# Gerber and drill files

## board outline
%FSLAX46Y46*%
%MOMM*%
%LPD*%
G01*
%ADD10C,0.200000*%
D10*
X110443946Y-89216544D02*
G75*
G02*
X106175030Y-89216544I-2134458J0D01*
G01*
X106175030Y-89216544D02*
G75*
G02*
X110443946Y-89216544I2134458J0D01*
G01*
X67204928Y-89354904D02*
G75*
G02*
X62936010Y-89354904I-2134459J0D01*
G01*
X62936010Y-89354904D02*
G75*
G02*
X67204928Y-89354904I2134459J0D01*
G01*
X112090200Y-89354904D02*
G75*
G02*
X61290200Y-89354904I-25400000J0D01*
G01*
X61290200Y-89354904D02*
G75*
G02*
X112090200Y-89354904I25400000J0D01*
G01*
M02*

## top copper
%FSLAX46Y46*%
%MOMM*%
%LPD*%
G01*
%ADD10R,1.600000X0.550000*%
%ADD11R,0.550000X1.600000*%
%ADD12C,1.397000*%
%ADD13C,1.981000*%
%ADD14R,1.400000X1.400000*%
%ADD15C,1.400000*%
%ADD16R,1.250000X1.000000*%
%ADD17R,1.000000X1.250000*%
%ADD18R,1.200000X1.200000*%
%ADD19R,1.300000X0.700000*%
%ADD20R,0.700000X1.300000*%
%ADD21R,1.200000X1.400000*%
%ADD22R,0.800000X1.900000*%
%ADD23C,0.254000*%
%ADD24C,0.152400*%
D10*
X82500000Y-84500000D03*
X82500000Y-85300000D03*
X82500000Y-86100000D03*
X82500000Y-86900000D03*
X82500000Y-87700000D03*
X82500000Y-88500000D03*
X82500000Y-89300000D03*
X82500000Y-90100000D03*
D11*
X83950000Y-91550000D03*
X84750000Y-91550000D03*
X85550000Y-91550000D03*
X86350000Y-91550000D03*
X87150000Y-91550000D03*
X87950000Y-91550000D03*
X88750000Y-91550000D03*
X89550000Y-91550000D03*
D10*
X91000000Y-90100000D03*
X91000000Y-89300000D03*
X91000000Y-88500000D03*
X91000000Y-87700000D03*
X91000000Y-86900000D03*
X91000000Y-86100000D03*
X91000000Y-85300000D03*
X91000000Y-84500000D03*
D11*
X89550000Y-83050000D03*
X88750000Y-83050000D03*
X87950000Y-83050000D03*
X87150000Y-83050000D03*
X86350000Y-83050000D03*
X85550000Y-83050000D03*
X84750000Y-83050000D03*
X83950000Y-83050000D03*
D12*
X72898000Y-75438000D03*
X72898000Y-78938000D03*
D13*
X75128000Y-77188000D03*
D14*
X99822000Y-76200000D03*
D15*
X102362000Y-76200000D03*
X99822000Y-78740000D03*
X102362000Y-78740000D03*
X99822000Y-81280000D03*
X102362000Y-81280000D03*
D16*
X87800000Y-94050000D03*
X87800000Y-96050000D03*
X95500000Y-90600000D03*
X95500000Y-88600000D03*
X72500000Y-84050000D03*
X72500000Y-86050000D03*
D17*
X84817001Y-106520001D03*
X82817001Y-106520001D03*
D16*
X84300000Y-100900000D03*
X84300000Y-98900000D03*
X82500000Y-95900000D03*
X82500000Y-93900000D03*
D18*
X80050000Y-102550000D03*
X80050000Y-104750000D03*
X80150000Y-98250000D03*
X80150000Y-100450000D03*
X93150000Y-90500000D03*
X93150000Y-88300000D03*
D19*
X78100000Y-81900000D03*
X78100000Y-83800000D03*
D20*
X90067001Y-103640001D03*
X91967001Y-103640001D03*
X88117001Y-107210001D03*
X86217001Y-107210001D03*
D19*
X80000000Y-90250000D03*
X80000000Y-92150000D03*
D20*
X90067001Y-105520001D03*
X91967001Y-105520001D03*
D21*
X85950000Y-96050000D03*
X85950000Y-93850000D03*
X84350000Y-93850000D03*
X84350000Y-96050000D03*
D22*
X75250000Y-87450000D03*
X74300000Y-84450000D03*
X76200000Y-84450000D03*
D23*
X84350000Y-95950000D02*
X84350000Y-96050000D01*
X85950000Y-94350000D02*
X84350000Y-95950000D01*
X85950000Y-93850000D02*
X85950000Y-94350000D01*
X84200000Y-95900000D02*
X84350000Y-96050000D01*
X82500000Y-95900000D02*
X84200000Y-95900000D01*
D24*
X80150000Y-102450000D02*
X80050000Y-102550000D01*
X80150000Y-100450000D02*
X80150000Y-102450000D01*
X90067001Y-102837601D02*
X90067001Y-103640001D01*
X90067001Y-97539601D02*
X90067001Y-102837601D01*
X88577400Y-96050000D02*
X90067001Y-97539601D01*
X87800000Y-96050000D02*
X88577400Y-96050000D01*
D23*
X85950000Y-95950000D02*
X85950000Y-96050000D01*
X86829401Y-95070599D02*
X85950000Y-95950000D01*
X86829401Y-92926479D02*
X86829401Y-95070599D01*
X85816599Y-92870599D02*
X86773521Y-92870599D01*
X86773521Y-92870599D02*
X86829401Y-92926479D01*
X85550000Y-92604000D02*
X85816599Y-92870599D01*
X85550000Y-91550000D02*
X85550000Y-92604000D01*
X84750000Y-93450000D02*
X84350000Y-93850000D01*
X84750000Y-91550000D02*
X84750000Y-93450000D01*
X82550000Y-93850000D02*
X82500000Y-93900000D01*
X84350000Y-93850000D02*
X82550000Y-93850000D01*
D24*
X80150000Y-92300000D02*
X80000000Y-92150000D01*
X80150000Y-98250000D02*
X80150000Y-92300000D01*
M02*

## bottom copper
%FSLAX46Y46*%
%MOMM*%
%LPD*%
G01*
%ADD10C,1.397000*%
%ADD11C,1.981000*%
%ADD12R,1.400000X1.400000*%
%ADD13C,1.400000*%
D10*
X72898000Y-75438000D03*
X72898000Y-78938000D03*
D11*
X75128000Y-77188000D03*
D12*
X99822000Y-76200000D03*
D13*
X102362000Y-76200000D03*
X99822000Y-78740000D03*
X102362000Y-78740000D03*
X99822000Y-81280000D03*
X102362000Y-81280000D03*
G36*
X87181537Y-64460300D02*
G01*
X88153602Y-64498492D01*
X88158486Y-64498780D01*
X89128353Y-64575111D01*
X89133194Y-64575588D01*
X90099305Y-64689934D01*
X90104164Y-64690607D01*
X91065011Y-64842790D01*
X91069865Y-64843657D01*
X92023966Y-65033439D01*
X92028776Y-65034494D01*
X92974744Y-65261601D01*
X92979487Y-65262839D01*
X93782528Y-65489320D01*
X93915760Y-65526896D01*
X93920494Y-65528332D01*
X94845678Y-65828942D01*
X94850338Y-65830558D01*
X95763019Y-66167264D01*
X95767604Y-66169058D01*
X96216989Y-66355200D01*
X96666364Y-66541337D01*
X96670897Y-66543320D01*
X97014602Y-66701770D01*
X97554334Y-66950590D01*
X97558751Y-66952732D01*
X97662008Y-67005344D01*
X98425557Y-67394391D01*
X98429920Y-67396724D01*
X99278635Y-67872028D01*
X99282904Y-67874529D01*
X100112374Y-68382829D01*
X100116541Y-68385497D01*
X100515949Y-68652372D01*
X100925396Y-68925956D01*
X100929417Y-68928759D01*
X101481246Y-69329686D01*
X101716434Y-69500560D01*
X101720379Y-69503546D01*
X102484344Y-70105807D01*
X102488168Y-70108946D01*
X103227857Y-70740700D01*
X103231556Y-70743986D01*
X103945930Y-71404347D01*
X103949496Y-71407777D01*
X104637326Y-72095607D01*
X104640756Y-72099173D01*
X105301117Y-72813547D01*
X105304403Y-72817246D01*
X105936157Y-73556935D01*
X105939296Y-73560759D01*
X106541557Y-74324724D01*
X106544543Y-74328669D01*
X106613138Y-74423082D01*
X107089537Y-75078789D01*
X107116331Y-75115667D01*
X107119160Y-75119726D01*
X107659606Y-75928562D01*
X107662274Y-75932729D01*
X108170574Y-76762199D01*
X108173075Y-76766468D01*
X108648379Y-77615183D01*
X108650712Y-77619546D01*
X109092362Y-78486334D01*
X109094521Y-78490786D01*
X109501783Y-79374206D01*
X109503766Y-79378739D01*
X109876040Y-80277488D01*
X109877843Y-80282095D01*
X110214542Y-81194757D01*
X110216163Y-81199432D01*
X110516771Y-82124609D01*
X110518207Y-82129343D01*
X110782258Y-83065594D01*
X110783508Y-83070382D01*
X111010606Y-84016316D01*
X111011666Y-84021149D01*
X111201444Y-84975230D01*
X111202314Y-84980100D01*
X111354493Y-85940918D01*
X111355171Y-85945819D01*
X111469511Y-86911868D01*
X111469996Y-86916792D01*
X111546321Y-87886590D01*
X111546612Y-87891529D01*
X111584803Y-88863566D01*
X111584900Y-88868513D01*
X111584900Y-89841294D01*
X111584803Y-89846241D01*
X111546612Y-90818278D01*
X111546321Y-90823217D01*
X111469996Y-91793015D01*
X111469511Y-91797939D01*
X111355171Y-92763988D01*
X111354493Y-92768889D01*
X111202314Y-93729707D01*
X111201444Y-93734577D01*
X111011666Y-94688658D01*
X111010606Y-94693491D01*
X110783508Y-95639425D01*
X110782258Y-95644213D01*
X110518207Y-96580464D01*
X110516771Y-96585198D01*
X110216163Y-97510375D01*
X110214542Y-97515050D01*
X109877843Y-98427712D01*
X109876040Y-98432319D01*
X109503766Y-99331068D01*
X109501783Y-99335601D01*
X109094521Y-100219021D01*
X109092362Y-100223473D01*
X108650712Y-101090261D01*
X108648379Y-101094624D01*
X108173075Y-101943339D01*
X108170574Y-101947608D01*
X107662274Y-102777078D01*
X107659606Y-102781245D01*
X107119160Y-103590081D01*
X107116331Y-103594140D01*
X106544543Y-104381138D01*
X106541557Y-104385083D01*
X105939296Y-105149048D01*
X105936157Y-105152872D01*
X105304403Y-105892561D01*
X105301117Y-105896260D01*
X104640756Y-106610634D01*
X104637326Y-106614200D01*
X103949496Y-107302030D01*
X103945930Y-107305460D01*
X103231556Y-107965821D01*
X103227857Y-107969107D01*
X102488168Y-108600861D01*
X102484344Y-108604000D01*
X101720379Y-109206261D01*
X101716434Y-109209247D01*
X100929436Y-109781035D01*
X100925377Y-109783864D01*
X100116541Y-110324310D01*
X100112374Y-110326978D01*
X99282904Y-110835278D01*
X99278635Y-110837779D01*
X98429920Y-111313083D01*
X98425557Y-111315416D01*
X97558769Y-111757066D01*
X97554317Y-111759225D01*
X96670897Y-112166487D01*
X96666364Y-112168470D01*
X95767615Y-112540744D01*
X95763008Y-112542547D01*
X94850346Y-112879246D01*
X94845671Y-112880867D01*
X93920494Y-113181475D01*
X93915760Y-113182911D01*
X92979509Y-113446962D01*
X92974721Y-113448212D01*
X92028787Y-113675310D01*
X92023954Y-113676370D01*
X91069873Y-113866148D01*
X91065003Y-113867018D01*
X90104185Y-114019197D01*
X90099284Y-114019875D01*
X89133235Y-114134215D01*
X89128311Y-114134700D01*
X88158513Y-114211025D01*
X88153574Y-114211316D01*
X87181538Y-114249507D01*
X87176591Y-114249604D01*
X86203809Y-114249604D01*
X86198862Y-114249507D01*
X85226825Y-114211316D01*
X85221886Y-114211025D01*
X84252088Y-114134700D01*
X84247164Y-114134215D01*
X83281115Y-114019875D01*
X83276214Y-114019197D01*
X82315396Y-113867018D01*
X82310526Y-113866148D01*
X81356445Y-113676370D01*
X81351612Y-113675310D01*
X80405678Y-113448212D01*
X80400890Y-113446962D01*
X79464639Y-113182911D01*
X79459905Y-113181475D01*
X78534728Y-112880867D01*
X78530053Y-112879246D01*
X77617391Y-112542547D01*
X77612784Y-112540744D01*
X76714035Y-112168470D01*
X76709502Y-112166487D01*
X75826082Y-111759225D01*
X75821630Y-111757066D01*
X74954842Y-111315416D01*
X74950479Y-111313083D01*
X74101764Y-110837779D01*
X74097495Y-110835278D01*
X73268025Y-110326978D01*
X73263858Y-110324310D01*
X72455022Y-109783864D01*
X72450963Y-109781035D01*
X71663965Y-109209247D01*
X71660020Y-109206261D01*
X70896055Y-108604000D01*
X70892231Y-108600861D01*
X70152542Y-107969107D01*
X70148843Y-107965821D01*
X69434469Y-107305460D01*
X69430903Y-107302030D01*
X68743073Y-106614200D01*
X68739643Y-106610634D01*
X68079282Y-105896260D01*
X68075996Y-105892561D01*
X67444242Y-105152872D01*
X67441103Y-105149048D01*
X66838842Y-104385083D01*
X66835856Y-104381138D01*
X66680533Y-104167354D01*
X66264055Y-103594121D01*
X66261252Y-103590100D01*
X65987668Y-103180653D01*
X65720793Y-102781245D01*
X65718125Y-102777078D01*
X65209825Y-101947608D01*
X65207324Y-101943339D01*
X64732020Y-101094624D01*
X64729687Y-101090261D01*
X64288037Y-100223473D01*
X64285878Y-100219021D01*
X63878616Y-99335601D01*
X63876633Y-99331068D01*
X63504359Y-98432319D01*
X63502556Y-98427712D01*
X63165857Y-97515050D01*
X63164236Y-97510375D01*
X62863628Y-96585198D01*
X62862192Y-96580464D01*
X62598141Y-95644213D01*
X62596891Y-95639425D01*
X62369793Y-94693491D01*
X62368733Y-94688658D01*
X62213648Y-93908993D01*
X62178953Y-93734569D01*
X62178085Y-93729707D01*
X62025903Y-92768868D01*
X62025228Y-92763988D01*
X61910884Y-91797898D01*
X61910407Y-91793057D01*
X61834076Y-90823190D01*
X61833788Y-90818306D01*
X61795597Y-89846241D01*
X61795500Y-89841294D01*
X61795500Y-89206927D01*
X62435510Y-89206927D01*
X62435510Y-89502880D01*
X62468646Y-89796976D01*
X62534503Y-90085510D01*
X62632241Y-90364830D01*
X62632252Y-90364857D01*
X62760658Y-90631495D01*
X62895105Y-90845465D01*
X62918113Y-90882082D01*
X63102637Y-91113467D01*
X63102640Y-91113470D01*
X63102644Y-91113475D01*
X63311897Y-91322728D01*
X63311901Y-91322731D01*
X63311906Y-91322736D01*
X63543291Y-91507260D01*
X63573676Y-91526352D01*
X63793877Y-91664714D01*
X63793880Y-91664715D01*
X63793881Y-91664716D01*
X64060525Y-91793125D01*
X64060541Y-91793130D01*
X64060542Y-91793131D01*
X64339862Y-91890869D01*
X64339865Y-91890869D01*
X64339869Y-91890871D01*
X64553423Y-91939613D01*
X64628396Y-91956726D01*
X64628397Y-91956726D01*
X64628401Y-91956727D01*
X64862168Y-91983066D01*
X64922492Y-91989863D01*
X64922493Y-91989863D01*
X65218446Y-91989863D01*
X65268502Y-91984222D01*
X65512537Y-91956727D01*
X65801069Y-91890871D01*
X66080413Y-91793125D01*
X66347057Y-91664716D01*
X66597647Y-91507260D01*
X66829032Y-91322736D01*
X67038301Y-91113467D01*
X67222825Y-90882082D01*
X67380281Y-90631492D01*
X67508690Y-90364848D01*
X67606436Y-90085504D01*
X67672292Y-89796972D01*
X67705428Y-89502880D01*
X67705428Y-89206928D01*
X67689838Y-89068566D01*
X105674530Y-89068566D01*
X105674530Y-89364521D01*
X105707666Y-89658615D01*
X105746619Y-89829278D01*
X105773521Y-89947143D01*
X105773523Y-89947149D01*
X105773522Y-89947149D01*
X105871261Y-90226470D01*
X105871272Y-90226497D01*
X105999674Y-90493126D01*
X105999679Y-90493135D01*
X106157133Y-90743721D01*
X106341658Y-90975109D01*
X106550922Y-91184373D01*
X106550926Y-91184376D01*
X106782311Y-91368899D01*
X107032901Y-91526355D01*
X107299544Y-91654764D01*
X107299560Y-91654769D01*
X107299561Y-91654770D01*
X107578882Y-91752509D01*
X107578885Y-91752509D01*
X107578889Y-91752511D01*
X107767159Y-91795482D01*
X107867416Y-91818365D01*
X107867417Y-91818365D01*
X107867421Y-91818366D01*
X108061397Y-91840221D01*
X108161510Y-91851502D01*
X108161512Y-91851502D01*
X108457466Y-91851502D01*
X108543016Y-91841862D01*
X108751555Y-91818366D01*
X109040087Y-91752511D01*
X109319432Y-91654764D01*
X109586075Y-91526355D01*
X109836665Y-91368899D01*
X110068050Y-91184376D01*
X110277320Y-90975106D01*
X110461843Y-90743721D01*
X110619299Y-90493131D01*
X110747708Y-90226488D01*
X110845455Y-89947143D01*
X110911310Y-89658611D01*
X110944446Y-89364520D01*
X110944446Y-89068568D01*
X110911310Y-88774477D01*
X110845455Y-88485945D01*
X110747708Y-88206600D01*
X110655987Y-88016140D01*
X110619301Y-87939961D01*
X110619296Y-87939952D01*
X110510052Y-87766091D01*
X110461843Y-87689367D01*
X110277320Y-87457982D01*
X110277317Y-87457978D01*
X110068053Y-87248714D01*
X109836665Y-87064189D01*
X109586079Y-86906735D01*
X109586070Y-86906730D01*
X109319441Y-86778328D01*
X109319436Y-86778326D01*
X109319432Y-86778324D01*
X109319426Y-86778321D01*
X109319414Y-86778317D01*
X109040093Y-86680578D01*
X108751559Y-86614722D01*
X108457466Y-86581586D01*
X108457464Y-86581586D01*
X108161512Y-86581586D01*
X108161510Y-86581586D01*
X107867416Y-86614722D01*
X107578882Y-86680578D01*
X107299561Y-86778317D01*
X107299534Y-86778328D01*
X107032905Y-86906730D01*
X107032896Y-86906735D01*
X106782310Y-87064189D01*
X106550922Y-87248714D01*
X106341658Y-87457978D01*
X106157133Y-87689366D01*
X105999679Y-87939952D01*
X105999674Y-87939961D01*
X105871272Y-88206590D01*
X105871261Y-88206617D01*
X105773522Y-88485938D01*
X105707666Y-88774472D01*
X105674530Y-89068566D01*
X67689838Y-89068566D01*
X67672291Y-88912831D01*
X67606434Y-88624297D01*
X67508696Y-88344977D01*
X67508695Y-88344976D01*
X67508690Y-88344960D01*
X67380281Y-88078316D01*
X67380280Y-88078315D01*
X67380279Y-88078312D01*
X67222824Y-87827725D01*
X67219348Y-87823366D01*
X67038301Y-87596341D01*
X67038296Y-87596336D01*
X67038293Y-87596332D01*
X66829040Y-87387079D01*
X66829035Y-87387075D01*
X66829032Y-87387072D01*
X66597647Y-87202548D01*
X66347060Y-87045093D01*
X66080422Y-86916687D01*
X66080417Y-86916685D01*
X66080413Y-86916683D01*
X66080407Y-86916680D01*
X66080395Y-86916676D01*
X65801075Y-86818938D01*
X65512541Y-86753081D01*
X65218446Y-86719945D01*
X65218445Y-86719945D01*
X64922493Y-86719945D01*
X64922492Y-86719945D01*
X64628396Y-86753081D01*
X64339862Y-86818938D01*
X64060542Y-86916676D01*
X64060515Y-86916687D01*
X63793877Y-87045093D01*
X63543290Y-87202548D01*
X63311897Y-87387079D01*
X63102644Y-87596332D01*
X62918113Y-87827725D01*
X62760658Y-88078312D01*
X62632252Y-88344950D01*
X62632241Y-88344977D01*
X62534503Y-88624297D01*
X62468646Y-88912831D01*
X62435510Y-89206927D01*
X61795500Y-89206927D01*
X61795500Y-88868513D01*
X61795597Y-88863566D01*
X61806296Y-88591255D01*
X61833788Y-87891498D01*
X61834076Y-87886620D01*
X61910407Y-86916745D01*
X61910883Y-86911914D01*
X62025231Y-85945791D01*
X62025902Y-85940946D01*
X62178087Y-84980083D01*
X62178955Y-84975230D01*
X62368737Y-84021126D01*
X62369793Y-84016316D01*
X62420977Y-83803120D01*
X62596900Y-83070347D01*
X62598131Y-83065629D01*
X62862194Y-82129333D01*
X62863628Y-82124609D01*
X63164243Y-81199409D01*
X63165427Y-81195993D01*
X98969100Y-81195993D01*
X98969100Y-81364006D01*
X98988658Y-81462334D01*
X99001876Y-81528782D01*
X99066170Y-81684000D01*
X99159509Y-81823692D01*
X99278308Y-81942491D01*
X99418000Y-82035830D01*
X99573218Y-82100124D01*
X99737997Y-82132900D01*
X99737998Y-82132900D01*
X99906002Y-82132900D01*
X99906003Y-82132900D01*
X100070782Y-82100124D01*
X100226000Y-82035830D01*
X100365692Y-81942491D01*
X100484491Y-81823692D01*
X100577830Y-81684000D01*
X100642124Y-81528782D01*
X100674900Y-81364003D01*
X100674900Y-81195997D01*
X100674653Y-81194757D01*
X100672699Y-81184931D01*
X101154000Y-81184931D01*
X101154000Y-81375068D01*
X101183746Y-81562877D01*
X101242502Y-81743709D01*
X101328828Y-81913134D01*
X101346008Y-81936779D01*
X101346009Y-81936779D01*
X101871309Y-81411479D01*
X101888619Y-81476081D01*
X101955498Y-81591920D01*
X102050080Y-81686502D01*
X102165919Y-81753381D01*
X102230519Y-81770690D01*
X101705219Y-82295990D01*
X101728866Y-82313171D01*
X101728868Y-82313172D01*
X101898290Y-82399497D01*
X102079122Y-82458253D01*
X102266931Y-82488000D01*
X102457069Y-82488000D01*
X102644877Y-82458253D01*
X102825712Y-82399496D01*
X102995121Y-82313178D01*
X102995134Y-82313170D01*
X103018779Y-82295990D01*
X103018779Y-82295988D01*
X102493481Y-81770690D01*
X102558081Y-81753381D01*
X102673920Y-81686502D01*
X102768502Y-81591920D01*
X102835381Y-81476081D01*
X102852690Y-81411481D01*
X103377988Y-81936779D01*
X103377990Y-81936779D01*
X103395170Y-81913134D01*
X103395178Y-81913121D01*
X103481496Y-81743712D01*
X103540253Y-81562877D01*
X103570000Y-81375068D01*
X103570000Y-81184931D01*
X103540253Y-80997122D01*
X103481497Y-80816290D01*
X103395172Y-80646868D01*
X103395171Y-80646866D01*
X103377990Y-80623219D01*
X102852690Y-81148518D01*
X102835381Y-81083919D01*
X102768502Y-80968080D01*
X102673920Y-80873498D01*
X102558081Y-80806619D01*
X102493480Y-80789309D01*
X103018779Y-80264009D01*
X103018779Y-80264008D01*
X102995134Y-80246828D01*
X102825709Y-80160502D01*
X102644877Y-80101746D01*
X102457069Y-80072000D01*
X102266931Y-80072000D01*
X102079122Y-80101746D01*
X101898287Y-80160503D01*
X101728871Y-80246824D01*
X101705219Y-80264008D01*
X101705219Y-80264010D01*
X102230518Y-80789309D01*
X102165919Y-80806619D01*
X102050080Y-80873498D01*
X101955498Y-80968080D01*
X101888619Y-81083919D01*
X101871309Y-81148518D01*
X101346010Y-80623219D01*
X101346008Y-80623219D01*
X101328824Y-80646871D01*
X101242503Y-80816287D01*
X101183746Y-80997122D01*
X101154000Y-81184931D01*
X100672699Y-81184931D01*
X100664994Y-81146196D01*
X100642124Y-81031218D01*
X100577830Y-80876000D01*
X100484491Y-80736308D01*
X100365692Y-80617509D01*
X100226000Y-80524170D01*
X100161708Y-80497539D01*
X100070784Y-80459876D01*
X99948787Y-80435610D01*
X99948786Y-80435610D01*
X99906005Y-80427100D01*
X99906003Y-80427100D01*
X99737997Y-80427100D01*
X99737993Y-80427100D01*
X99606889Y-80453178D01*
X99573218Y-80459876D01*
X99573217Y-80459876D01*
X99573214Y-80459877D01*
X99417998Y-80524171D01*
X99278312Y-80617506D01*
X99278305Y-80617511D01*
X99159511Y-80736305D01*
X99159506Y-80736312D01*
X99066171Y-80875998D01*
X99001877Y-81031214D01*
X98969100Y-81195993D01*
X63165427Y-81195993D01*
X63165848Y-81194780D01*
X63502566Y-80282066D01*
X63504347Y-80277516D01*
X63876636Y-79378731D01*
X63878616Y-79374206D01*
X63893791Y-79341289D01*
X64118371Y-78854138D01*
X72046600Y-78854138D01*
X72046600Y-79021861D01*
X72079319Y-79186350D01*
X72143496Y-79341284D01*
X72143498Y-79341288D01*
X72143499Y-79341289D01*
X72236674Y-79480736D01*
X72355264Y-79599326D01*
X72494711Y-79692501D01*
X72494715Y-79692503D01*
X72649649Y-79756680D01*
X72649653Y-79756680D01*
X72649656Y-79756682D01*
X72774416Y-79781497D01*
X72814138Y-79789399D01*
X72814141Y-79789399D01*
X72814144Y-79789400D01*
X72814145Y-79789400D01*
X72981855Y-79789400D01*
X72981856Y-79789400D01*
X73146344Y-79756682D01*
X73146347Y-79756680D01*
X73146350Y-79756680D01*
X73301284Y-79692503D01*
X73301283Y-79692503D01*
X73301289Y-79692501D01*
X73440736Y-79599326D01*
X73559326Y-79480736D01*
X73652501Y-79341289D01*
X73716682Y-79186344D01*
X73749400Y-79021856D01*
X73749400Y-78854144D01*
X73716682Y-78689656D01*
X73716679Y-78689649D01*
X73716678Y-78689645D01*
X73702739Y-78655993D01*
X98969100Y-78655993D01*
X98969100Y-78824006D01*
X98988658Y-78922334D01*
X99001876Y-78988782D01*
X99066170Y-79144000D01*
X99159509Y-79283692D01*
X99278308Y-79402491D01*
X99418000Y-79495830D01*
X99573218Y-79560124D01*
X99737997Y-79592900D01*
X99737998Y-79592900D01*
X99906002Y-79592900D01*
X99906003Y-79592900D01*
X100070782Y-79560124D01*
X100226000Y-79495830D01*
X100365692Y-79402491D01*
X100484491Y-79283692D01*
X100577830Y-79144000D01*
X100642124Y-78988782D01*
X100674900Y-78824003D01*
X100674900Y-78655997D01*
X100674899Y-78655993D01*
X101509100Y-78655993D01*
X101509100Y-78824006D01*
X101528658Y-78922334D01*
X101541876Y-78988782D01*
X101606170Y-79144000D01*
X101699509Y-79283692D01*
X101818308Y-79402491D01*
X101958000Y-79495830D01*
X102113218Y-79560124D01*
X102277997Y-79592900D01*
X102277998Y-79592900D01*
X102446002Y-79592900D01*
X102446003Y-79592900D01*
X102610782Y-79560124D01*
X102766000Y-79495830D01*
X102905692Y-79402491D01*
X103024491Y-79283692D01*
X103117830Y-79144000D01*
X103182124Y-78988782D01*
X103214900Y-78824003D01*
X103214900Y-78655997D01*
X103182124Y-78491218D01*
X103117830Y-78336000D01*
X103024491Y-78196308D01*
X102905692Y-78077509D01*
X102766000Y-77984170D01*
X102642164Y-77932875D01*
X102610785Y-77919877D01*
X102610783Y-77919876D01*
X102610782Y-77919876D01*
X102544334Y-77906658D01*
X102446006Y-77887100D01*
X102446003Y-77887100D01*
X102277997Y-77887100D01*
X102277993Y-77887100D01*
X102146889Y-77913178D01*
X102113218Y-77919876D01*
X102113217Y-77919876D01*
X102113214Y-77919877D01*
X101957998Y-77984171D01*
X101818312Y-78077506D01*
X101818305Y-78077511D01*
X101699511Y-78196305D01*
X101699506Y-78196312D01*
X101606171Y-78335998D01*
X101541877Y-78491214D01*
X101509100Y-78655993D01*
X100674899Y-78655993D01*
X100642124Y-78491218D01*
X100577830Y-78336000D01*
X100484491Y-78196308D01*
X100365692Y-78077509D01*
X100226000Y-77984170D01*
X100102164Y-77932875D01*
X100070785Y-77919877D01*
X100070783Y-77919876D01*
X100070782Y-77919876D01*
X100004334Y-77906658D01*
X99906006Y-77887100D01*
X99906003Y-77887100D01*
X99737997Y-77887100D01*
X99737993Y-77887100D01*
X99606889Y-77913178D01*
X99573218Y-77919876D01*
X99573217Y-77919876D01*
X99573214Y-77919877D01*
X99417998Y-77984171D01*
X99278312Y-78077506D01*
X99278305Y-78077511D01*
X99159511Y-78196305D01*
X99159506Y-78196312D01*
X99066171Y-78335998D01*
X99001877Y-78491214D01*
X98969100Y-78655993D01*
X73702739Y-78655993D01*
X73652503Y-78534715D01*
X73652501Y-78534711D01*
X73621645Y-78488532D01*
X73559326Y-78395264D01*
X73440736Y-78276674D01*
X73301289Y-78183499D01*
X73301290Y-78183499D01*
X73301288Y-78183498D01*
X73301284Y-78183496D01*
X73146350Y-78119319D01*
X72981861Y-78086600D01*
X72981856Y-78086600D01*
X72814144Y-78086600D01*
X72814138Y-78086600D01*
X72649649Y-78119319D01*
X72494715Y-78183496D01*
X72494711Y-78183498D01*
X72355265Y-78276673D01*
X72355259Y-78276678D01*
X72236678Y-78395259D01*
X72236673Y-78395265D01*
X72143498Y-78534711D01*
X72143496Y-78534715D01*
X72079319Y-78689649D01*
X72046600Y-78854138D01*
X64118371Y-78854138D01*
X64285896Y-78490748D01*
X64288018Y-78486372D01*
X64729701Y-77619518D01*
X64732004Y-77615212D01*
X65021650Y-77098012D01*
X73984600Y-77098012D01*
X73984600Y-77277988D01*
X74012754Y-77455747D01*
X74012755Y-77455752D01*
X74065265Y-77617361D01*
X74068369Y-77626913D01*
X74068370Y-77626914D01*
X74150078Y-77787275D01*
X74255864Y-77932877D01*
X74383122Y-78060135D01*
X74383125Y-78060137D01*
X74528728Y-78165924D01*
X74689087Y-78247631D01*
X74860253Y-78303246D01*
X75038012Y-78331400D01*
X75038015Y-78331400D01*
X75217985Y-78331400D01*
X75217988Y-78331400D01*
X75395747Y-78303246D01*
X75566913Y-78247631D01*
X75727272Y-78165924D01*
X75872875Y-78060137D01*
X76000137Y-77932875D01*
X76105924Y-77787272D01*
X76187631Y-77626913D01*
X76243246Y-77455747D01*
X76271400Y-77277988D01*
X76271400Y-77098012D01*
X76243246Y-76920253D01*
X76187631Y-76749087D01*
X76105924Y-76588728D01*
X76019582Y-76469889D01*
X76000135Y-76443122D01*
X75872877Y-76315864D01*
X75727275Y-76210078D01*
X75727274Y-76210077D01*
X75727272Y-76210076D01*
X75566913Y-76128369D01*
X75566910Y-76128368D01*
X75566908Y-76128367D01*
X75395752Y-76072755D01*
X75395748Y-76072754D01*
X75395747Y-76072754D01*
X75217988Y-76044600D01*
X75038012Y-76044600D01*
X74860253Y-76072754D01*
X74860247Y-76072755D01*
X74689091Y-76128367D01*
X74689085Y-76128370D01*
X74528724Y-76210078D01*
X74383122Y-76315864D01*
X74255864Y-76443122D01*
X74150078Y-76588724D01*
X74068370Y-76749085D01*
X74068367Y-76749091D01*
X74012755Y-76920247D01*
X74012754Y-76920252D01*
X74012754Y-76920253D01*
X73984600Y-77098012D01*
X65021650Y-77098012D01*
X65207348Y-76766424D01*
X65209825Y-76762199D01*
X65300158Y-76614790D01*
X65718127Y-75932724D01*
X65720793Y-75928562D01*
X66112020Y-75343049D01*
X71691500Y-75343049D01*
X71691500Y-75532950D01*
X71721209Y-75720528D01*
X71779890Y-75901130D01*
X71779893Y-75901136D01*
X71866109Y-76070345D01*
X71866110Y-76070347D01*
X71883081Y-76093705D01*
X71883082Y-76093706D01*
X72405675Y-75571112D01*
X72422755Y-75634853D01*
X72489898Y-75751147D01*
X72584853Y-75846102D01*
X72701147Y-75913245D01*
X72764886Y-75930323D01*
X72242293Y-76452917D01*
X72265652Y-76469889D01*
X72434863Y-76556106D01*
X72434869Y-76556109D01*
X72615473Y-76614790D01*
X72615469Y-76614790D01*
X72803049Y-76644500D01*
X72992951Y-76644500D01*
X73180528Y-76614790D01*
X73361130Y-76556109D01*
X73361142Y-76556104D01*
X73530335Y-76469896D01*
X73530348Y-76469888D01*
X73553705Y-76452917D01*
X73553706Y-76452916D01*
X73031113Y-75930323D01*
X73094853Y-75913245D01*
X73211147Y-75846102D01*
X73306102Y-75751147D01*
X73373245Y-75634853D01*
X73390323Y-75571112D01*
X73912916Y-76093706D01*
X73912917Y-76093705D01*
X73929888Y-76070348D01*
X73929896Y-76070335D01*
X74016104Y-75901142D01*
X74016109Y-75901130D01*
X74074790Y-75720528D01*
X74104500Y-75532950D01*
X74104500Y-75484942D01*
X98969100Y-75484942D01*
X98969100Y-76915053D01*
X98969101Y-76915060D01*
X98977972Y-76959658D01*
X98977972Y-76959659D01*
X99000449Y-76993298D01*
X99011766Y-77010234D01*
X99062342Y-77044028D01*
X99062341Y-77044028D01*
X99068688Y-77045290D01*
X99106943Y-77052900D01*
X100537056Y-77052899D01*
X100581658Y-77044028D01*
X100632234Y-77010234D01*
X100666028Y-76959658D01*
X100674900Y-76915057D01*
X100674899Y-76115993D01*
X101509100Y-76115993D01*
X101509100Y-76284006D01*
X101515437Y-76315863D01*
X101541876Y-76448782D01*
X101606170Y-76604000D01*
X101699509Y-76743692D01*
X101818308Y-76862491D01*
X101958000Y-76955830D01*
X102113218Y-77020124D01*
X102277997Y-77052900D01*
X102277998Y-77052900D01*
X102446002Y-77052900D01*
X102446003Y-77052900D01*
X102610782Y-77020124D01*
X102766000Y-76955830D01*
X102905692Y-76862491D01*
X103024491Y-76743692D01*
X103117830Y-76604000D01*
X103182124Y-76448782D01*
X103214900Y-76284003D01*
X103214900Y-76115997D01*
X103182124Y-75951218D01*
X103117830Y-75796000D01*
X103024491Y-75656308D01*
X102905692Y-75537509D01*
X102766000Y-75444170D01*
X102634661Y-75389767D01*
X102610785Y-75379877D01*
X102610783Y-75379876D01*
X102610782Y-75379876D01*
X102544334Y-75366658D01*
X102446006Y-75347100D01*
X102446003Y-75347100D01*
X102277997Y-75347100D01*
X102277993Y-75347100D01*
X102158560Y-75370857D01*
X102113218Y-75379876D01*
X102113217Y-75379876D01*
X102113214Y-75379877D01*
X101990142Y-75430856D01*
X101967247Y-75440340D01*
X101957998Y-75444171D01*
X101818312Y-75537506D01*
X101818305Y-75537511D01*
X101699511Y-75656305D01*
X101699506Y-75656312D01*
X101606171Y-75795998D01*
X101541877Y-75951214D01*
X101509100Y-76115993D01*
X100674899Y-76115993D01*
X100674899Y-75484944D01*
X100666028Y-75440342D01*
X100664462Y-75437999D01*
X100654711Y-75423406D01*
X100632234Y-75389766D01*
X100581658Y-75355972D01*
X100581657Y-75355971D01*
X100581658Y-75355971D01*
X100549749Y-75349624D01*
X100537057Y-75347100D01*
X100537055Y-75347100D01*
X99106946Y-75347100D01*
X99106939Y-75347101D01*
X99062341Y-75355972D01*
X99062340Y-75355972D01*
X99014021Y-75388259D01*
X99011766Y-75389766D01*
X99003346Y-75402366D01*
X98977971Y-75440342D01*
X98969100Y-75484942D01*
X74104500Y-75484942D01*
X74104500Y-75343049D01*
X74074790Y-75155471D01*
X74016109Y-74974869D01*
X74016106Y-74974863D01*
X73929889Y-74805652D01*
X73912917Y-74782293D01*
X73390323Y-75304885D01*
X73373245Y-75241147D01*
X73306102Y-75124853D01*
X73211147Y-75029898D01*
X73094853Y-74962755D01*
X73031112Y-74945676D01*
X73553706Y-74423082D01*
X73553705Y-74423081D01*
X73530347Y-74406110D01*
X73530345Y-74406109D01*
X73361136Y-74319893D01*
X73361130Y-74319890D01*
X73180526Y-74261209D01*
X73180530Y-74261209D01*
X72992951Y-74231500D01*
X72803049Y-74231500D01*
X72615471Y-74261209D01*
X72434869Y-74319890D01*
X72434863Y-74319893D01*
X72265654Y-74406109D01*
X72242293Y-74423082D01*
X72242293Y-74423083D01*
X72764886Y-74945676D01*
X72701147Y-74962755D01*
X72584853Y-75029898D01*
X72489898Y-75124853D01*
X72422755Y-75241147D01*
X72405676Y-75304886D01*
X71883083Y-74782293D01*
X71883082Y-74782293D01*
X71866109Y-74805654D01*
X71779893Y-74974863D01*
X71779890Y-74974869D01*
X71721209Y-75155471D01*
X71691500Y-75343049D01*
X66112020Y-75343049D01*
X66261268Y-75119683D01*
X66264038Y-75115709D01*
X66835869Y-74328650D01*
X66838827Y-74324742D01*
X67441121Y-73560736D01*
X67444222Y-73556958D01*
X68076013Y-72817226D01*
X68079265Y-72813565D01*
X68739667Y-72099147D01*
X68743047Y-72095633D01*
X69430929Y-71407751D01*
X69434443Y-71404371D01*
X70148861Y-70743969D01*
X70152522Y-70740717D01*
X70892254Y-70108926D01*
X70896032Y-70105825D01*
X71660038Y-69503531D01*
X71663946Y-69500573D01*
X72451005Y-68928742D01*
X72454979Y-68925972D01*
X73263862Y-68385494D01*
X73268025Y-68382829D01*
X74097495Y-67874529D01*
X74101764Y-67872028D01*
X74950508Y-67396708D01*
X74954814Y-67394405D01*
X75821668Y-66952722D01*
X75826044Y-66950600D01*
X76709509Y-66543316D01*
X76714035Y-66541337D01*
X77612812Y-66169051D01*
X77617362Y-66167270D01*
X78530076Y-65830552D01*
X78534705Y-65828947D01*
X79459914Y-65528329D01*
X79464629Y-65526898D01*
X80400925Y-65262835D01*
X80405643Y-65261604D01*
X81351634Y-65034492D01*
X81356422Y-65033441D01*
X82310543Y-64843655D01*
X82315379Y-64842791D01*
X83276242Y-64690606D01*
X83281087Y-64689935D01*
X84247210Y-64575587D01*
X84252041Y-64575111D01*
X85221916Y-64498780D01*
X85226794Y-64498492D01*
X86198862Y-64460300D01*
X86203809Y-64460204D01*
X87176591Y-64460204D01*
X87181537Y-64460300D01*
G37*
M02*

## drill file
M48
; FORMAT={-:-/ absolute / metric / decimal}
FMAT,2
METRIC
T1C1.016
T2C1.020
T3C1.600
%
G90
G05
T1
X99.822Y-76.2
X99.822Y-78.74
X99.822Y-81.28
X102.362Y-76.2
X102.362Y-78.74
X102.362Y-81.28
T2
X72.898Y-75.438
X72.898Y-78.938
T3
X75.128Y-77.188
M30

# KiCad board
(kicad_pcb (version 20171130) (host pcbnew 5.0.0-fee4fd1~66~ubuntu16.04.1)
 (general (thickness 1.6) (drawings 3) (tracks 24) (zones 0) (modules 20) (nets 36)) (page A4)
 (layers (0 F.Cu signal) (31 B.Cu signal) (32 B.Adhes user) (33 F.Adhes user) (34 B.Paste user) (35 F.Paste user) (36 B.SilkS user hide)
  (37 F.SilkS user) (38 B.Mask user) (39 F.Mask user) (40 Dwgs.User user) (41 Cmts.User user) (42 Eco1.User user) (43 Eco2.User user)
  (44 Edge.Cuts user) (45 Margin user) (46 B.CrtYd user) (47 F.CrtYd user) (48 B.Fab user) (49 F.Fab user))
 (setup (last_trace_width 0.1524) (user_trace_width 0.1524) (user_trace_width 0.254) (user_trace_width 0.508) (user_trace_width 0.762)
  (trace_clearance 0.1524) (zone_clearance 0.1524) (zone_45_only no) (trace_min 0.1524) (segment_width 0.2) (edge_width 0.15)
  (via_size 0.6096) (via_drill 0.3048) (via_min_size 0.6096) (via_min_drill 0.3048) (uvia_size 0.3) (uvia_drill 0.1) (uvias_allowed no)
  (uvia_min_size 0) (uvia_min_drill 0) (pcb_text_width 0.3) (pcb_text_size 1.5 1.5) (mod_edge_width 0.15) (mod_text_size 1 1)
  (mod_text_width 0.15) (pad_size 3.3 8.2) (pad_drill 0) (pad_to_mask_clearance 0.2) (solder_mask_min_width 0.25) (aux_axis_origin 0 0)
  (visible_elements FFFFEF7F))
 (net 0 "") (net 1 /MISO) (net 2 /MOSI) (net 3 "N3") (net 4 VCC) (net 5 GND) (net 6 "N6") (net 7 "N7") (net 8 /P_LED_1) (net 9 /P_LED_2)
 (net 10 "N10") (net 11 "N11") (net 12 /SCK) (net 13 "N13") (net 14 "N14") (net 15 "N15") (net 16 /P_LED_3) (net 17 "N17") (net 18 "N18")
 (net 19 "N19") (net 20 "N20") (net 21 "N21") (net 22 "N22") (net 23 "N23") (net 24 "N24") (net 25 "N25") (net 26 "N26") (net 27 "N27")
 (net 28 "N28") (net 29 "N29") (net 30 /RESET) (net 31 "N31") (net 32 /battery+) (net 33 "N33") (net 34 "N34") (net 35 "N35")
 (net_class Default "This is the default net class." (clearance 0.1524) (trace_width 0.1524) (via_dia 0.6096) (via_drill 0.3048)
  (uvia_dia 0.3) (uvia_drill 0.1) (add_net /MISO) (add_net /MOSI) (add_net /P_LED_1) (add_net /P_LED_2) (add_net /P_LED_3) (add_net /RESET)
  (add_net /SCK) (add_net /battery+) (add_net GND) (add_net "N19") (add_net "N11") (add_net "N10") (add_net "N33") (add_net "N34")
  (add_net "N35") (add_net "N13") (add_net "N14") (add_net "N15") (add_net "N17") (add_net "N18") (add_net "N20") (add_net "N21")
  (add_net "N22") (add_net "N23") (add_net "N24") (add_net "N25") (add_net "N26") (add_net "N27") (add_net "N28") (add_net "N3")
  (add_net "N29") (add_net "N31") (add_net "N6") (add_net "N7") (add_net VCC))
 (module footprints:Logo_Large (layer B.Cu) (at 86.614 88.9 180)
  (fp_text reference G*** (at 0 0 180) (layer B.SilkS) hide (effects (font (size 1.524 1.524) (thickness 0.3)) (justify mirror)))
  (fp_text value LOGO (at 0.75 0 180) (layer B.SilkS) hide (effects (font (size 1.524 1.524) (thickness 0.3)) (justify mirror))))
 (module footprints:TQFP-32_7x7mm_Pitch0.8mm (layer F.Cu) (at 86.75 87.3)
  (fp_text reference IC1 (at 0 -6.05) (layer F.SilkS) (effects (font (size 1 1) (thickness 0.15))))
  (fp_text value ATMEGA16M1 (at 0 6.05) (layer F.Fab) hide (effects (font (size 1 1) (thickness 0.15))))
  (pad 1 smd rect (at -4.25 -2.8) (size 1.6 0.55) (layers F.Cu F.Paste F.Mask) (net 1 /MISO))
  (pad 2 smd rect (at -4.25 -2) (size 1.6 0.55) (layers F.Cu F.Paste F.Mask) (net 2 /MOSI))
  (pad 3 smd rect (at -4.25 -1.2) (size 1.6 0.55) (layers F.Cu F.Paste F.Mask) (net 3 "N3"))
  (pad 4 smd rect (at -4.25 -0.4) (size 1.6 0.55) (layers F.Cu F.Paste F.Mask) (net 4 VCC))
  (pad 5 smd rect (at -4.25 0.4) (size 1.6 0.55) (layers F.Cu F.Paste F.Mask) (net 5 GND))
  (pad 6 smd rect (at -4.25 1.2) (size 1.6 0.55) (layers F.Cu F.Paste F.Mask) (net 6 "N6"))
  (pad 7 smd rect (at -4.25 2) (size 1.6 0.55) (layers F.Cu F.Paste F.Mask) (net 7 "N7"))
  (pad 8 smd rect (at -4.25 2.8) (size 1.6 0.55) (layers F.Cu F.Paste F.Mask) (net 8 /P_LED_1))
  (pad 9 smd rect (at -2.8 4.25 90) (size 1.6 0.55) (layers F.Cu F.Paste F.Mask) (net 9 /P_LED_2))
  (pad 10 smd rect (at -2 4.25 90) (size 1.6 0.55) (layers F.Cu F.Paste F.Mask) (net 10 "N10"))
  (pad 11 smd rect (at -1.2 4.25 90) (size 1.6 0.55) (layers F.Cu F.Paste F.Mask) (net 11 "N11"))
  (pad 12 smd rect (at -0.4 4.25 90) (size 1.6 0.55) (layers F.Cu F.Paste F.Mask) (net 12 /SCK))
  (pad 13 smd rect (at 0.4 4.25 90) (size 1.6 0.55) (layers F.Cu F.Paste F.Mask) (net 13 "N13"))
  (pad 14 smd rect (at 1.2 4.25 90) (size 1.6 0.55) (layers F.Cu F.Paste F.Mask) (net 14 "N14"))
  (pad 15 smd rect (at 2 4.25 90) (size 1.6 0.55) (layers F.Cu F.Paste F.Mask) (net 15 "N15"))
  (pad 16 smd rect (at 2.8 4.25 90) (size 1.6 0.55) (layers F.Cu F.Paste F.Mask) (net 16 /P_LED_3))
  (pad 17 smd rect (at 4.25 2.8) (size 1.6 0.55) (layers F.Cu F.Paste F.Mask) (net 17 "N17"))
  (pad 18 smd rect (at 4.25 2) (size 1.6 0.55) (layers F.Cu F.Paste F.Mask) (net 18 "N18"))
  (pad 19 smd rect (at 4.25 1.2) (size 1.6 0.55) (layers F.Cu F.Paste F.Mask) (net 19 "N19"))
  (pad 20 smd rect (at 4.25 0.4) (size 1.6 0.55) (layers F.Cu F.Paste F.Mask) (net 5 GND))
  (pad 21 smd rect (at 4.25 -0.4) (size 1.6 0.55) (layers F.Cu F.Paste F.Mask) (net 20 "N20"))
  (pad 22 smd rect (at 4.25 -1.2) (size 1.6 0.55) (layers F.Cu F.Paste F.Mask) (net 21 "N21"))
  (pad 23 smd rect (at 4.25 -2) (size 1.6 0.55) (layers F.Cu F.Paste F.Mask) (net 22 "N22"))
  (pad 24 smd rect (at 4.25 -2.8) (size 1.6 0.55) (layers F.Cu F.Paste F.Mask) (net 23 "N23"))
  (pad 25 smd rect (at 2.8 -4.25 90) (size 1.6 0.55) (layers F.Cu F.Paste F.Mask) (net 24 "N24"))
  (pad 26 smd rect (at 2 -4.25 90) (size 1.6 0.55) (layers F.Cu F.Paste F.Mask) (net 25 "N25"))
  (pad 27 smd rect (at 1.2 -4.25 90) (size 1.6 0.55) (layers F.Cu F.Paste F.Mask) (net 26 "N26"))
  (pad 28 smd rect (at 0.4 -4.25 90) (size 1.6 0.55) (layers F.Cu F.Paste F.Mask) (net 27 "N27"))
  (pad 29 smd rect (at -0.4 -4.25 90) (size 1.6 0.55) (layers F.Cu F.Paste F.Mask) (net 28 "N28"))
  (pad 30 smd rect (at -1.2 -4.25 90) (size 1.6 0.55) (layers F.Cu F.Paste F.Mask) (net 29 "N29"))
  (pad 31 smd rect (at -2 -4.25 90) (size 1.6 0.55) (layers F.Cu F.Paste F.Mask) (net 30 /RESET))
  (pad 32 smd rect (at -2.8 -4.25 90) (size 1.6 0.55) (layers F.Cu F.Paste F.Mask) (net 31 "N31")))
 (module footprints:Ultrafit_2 (layer F.Cu) (at 72.898 75.438)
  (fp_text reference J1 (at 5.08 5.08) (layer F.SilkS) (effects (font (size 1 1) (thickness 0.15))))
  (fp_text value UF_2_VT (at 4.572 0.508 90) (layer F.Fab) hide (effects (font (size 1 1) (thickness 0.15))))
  (pad 2 thru_hole circle (at 0 0) (size 1.397 1.397) (drill 1.02) (layers *.Cu *.Mask) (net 5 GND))
  (pad 1 thru_hole circle (at 0 3.5) (size 1.397 1.397) (drill 1.02) (layers *.Cu *.Mask) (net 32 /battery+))
  (pad "" thru_hole circle (at 2.23 1.75) (size 1.981 1.981) (drill 1.6) (layers *.Cu *.Mask)))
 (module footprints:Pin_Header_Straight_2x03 (layer F.Cu) (at 99.822 76.2)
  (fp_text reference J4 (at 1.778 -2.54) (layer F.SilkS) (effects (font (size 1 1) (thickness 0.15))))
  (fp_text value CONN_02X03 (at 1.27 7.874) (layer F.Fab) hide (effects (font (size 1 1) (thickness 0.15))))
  (pad 1 thru_hole rect (at 0 0) (size 1.4 1.4) (drill 1.016) (layers *.Cu *.Mask) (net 1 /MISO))
  (pad 2 thru_hole circle (at 2.54 0) (size 1.4 1.4) (drill 1.016) (layers *.Cu *.Mask) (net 4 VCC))
  (pad 3 thru_hole circle (at 0 2.54) (size 1.4 1.4) (drill 1.016) (layers *.Cu *.Mask) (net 12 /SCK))
  (pad 4 thru_hole circle (at 2.54 2.54) (size 1.4 1.4) (drill 1.016) (layers *.Cu *.Mask) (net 2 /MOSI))
  (pad 5 thru_hole circle (at 0 5.08) (size 1.4 1.4) (drill 1.016) (layers *.Cu *.Mask) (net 30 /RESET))
  (pad 6 thru_hole circle (at 2.54 5.08) (size 1.4 1.4) (drill 1.016) (layers *.Cu *.Mask) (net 5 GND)))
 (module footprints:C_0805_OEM (layer F.Cu) (at 87.8 95.05 90)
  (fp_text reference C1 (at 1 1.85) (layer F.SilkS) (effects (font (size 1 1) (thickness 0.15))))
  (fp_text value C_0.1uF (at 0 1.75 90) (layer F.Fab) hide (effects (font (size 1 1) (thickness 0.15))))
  (pad 2 smd rect (at 1 0 90) (size 1 1.25) (layers F.Cu F.Paste F.Mask) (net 5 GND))
  (pad 1 smd rect (at -1 0 90) (size 1 1.25) (layers F.Cu F.Paste F.Mask) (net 4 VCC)))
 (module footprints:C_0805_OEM (layer F.Cu) (at 95.5 89.6 90)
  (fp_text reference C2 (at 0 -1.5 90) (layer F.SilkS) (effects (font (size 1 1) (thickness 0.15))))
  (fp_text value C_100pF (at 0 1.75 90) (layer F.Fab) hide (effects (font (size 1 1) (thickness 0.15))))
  (pad 1 smd rect (at -1 0 90) (size 1 1.25) (layers F.Cu F.Paste F.Mask) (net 19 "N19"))
  (pad 2 smd rect (at 1 0 90) (size 1 1.25) (layers F.Cu F.Paste F.Mask) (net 5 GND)))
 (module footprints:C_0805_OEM (layer F.Cu) (at 72.5 85.05 270)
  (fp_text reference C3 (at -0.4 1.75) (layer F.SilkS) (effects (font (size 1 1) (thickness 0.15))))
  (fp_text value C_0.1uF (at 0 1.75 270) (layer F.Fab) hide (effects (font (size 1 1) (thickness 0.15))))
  (pad 1 smd rect (at -1 0 270) (size 1 1.25) (layers F.Cu F.Paste F.Mask) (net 32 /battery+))
  (pad 2 smd rect (at 1 0 270) (size 1 1.25) (layers F.Cu F.Paste F.Mask) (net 5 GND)))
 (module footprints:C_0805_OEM (layer F.Cu) (at 83.817001 106.520001)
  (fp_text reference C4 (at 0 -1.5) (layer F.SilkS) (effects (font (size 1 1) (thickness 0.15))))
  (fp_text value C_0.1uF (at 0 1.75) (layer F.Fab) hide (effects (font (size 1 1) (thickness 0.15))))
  (pad 2 smd rect (at 1 0) (size 1 1.25) (layers F.Cu F.Paste F.Mask) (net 5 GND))
  (pad 1 smd rect (at -1 0) (size 1 1.25) (layers F.Cu F.Paste F.Mask) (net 4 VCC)))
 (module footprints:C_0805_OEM (layer F.Cu) (at 84.3 99.9 90)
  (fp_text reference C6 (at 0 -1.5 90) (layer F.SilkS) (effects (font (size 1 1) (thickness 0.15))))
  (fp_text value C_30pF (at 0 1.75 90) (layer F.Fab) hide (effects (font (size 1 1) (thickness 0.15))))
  (pad 1 smd rect (at -1 0 90) (size 1 1.25) (layers F.Cu F.Paste F.Mask) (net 11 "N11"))
  (pad 2 smd rect (at 1 0 90) (size 1 1.25) (layers F.Cu F.Paste F.Mask) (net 5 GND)))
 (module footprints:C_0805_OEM (layer F.Cu) (at 82.5 94.9 270)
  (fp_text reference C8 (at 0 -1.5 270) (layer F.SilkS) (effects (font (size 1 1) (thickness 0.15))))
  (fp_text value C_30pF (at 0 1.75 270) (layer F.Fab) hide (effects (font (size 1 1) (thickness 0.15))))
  (pad 2 smd rect (at 1 0 270) (size 1 1.25) (layers F.Cu F.Paste F.Mask) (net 5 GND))
  (pad 1 smd rect (at -1 0 270) (size 1 1.25) (layers F.Cu F.Paste F.Mask) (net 10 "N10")))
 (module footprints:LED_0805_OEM (layer F.Cu) (at 80.05 103.65 270)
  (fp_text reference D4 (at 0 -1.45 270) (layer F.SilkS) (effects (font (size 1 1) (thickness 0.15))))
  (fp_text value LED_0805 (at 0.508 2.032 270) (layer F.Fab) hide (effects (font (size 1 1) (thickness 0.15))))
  (pad 1 smd rect (at -1.1 0 90) (size 1.2 1.2) (layers F.Cu F.Paste F.Mask) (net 5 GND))
  (pad 2 smd rect (at 1.1 0 90) (size 1.2 1.2) (layers F.Cu F.Paste F.Mask) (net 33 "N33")))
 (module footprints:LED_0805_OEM (layer F.Cu) (at 80.15 99.35 90)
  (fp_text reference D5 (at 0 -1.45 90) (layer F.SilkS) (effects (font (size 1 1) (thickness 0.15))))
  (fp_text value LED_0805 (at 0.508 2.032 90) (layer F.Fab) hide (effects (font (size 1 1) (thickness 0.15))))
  (pad 2 smd rect (at 1.1 0 270) (size 1.2 1.2) (layers F.Cu F.Paste F.Mask) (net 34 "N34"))
  (pad 1 smd rect (at -1.1 0 270) (size 1.2 1.2) (layers F.Cu F.Paste F.Mask) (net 5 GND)))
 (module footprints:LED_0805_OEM (layer F.Cu) (at 93.15 89.4 270)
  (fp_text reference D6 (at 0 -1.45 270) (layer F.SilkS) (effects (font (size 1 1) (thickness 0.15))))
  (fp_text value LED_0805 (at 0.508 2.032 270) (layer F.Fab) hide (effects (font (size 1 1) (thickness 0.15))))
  (pad 2 smd rect (at 1.1 0 90) (size 1.2 1.2) (layers F.Cu F.Paste F.Mask) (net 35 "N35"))
  (pad 1 smd rect (at -1.1 0 90) (size 1.2 1.2) (layers F.Cu F.Paste F.Mask) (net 5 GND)))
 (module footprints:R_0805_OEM (layer F.Cu) (at 78.1 82.85 90)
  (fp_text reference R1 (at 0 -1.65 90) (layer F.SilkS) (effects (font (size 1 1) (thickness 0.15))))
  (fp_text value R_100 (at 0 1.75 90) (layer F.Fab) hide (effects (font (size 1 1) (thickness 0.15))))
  (pad 2 smd rect (at 0.95 0 90) (size 0.7 1.3) (layers F.Cu F.Paste F.Mask) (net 19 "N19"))
  (pad 1 smd rect (at -0.95 0 90) (size 0.7 1.3) (layers F.Cu F.Paste F.Mask) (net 4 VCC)))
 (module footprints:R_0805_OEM (layer F.Cu) (at 91.017001 103.640001)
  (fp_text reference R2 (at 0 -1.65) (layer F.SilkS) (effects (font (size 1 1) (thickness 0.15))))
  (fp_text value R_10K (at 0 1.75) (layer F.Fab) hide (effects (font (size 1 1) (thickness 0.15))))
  (pad 1 smd rect (at -0.95 0) (size 0.7 1.3) (layers F.Cu F.Paste F.Mask) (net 4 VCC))
  (pad 2 smd rect (at 0.95 0) (size 0.7 1.3) (layers F.Cu F.Paste F.Mask) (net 30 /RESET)))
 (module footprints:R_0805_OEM (layer F.Cu) (at 87.167001 107.210001)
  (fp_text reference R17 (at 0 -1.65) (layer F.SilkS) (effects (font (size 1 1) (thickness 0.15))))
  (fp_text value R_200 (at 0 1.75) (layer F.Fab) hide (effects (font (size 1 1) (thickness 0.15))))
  (pad 2 smd rect (at 0.95 0) (size 0.7 1.3) (layers F.Cu F.Paste F.Mask) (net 33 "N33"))
  (pad 1 smd rect (at -0.95 0) (size 0.7 1.3) (layers F.Cu F.Paste F.Mask) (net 16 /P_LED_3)))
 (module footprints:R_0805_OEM (layer F.Cu) (at 80 91.2 270)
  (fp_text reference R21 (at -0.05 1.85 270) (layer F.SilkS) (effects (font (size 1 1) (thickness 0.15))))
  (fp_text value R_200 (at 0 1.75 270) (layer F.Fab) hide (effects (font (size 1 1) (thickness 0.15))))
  (pad 1 smd rect (at -0.95 0 270) (size 0.7 1.3) (layers F.Cu F.Paste F.Mask) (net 8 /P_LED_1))
  (pad 2 smd rect (at 0.95 0 270) (size 0.7 1.3) (layers F.Cu F.Paste F.Mask) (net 34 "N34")))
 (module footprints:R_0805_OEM (layer F.Cu) (at 91.017001 105.520001)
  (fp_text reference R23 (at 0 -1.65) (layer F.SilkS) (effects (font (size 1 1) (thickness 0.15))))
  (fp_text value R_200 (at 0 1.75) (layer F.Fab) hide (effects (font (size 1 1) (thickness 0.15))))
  (pad 1 smd rect (at -0.95 0) (size 0.7 1.3) (layers F.Cu F.Paste F.Mask) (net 9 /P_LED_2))
  (pad 2 smd rect (at 0.95 0) (size 0.7 1.3) (layers F.Cu F.Paste F.Mask) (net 35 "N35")))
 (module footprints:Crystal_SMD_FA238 (layer F.Cu) (at 85.15 94.95 90)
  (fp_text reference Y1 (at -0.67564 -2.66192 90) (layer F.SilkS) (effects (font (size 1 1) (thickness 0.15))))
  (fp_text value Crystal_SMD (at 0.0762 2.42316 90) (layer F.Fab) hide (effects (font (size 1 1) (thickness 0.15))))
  (pad 1 smd rect (at -1.1 0.8 90) (size 1.4 1.2) (layers F.Cu F.Mask) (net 11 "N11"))
  (pad 2 smd rect (at 1.1 0.8 90) (size 1.4 1.2) (layers F.Cu F.Mask) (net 5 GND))
  (pad 3 smd rect (at 1.1 -0.8 90) (size 1.4 1.2) (layers F.Cu F.Mask) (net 10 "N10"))
  (pad 4 smd rect (at -1.1 -0.8 90) (size 1.4 1.2) (layers F.Cu F.Mask) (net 5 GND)))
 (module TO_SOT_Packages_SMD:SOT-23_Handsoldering (layer F.Cu) (at 75.25 85.95 270)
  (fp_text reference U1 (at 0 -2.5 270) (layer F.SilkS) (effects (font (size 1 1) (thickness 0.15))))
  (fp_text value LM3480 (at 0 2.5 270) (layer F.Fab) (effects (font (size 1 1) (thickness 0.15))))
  (pad 3 smd rect (at 1.5 0 270) (size 1.9 0.8) (layers F.Cu F.Paste F.Mask) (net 5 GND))
  (pad 2 smd rect (at -1.5 0.95 270) (size 1.9 0.8) (layers F.Cu F.Paste F.Mask) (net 32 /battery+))
  (pad 1 smd rect (at -1.5 -0.95 270) (size 1.9 0.8) (layers F.Cu F.Paste F.Mask) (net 4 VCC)))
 (gr_circle (center 108.309488 89.216544) (end 110.443946 89.216544) (layer Edge.Cuts) (width 0.2))
 (gr_circle (center 65.070469 89.354904) (end 67.204928 89.354904) (layer Edge.Cuts) (width 0.2))
 (gr_circle (center 86.6902 89.354904) (end 112.0902 89.354904) (layer Edge.Cuts) (width 0.2))
 (segment (start 84.35 95.95) (end 84.35 96.05) (width 0.254) (layer F.Cu) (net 5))
 (segment (start 85.95 94.35) (end 84.35 95.95) (width 0.254) (layer F.Cu) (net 5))
 (segment (start 85.95 93.85) (end 85.95 94.35) (width 0.254) (layer F.Cu) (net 5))
 (segment (start 84.2 95.9) (end 84.35 96.05) (width 0.254) (layer F.Cu) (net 5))
 (segment (start 82.5 95.9) (end 84.2 95.9) (width 0.254) (layer F.Cu) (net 5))
 (segment (start 80.15 102.45) (end 80.05 102.55) (width 0.1524) (layer F.Cu) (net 5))
 (segment (start 80.15 100.45) (end 80.15 102.45) (width 0.1524) (layer F.Cu) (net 5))
 (segment (start 90.067001 102.837601) (end 90.067001 103.640001) (width 0.1524) (layer F.Cu) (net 4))
 (segment (start 90.067001 97.539601) (end 90.067001 102.837601) (width 0.1524) (layer F.Cu) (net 4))
 (segment (start 88.5774 96.05) (end 90.067001 97.539601) (width 0.1524) (layer F.Cu) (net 4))
 (segment (start 87.8 96.05) (end 88.5774 96.05) (width 0.1524) (layer F.Cu) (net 4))
 (segment (start 85.95 95.95) (end 85.95 96.05) (width 0.254) (layer F.Cu) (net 11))
 (segment (start 86.829401 95.070599) (end 85.95 95.95) (width 0.254) (layer F.Cu) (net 11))
 (segment (start 86.829401 92.926479) (end 86.829401 95.070599) (width 0.254) (layer F.Cu) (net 11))
 (segment (start 85.816599 92.870599) (end 86.773521 92.870599) (width 0.254) (layer F.Cu) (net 11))
 (segment (start 86.773521 92.870599) (end 86.829401 92.926479) (width 0.254) (layer F.Cu) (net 11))
 (segment (start 85.55 92.604) (end 85.816599 92.870599) (width 0.254) (layer F.Cu) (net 11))
 (segment (start 85.55 91.55) (end 85.55 92.604) (width 0.254) (layer F.Cu) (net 11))
 (segment (start 84.75 93.45) (end 84.35 93.85) (width 0.254) (layer F.Cu) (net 10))
 (segment (start 84.75 91.55) (end 84.75 93.45) (width 0.254) (layer F.Cu) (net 10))
 (segment (start 82.55 93.85) (end 82.5 93.9) (width 0.254) (layer F.Cu) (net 10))
 (segment (start 84.35 93.85) (end 82.55 93.85) (width 0.254) (layer F.Cu) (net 10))
 (segment (start 80.15 92.3) (end 80 92.15) (width 0.1524) (layer F.Cu) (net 34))
 (segment (start 80.15 98.25) (end 80.15 92.3) (width 0.1524) (layer F.Cu) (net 34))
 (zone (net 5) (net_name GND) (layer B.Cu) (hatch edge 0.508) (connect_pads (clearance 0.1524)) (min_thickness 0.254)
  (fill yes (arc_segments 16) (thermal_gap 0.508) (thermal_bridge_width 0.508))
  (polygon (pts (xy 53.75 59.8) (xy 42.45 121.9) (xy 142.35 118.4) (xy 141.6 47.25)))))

